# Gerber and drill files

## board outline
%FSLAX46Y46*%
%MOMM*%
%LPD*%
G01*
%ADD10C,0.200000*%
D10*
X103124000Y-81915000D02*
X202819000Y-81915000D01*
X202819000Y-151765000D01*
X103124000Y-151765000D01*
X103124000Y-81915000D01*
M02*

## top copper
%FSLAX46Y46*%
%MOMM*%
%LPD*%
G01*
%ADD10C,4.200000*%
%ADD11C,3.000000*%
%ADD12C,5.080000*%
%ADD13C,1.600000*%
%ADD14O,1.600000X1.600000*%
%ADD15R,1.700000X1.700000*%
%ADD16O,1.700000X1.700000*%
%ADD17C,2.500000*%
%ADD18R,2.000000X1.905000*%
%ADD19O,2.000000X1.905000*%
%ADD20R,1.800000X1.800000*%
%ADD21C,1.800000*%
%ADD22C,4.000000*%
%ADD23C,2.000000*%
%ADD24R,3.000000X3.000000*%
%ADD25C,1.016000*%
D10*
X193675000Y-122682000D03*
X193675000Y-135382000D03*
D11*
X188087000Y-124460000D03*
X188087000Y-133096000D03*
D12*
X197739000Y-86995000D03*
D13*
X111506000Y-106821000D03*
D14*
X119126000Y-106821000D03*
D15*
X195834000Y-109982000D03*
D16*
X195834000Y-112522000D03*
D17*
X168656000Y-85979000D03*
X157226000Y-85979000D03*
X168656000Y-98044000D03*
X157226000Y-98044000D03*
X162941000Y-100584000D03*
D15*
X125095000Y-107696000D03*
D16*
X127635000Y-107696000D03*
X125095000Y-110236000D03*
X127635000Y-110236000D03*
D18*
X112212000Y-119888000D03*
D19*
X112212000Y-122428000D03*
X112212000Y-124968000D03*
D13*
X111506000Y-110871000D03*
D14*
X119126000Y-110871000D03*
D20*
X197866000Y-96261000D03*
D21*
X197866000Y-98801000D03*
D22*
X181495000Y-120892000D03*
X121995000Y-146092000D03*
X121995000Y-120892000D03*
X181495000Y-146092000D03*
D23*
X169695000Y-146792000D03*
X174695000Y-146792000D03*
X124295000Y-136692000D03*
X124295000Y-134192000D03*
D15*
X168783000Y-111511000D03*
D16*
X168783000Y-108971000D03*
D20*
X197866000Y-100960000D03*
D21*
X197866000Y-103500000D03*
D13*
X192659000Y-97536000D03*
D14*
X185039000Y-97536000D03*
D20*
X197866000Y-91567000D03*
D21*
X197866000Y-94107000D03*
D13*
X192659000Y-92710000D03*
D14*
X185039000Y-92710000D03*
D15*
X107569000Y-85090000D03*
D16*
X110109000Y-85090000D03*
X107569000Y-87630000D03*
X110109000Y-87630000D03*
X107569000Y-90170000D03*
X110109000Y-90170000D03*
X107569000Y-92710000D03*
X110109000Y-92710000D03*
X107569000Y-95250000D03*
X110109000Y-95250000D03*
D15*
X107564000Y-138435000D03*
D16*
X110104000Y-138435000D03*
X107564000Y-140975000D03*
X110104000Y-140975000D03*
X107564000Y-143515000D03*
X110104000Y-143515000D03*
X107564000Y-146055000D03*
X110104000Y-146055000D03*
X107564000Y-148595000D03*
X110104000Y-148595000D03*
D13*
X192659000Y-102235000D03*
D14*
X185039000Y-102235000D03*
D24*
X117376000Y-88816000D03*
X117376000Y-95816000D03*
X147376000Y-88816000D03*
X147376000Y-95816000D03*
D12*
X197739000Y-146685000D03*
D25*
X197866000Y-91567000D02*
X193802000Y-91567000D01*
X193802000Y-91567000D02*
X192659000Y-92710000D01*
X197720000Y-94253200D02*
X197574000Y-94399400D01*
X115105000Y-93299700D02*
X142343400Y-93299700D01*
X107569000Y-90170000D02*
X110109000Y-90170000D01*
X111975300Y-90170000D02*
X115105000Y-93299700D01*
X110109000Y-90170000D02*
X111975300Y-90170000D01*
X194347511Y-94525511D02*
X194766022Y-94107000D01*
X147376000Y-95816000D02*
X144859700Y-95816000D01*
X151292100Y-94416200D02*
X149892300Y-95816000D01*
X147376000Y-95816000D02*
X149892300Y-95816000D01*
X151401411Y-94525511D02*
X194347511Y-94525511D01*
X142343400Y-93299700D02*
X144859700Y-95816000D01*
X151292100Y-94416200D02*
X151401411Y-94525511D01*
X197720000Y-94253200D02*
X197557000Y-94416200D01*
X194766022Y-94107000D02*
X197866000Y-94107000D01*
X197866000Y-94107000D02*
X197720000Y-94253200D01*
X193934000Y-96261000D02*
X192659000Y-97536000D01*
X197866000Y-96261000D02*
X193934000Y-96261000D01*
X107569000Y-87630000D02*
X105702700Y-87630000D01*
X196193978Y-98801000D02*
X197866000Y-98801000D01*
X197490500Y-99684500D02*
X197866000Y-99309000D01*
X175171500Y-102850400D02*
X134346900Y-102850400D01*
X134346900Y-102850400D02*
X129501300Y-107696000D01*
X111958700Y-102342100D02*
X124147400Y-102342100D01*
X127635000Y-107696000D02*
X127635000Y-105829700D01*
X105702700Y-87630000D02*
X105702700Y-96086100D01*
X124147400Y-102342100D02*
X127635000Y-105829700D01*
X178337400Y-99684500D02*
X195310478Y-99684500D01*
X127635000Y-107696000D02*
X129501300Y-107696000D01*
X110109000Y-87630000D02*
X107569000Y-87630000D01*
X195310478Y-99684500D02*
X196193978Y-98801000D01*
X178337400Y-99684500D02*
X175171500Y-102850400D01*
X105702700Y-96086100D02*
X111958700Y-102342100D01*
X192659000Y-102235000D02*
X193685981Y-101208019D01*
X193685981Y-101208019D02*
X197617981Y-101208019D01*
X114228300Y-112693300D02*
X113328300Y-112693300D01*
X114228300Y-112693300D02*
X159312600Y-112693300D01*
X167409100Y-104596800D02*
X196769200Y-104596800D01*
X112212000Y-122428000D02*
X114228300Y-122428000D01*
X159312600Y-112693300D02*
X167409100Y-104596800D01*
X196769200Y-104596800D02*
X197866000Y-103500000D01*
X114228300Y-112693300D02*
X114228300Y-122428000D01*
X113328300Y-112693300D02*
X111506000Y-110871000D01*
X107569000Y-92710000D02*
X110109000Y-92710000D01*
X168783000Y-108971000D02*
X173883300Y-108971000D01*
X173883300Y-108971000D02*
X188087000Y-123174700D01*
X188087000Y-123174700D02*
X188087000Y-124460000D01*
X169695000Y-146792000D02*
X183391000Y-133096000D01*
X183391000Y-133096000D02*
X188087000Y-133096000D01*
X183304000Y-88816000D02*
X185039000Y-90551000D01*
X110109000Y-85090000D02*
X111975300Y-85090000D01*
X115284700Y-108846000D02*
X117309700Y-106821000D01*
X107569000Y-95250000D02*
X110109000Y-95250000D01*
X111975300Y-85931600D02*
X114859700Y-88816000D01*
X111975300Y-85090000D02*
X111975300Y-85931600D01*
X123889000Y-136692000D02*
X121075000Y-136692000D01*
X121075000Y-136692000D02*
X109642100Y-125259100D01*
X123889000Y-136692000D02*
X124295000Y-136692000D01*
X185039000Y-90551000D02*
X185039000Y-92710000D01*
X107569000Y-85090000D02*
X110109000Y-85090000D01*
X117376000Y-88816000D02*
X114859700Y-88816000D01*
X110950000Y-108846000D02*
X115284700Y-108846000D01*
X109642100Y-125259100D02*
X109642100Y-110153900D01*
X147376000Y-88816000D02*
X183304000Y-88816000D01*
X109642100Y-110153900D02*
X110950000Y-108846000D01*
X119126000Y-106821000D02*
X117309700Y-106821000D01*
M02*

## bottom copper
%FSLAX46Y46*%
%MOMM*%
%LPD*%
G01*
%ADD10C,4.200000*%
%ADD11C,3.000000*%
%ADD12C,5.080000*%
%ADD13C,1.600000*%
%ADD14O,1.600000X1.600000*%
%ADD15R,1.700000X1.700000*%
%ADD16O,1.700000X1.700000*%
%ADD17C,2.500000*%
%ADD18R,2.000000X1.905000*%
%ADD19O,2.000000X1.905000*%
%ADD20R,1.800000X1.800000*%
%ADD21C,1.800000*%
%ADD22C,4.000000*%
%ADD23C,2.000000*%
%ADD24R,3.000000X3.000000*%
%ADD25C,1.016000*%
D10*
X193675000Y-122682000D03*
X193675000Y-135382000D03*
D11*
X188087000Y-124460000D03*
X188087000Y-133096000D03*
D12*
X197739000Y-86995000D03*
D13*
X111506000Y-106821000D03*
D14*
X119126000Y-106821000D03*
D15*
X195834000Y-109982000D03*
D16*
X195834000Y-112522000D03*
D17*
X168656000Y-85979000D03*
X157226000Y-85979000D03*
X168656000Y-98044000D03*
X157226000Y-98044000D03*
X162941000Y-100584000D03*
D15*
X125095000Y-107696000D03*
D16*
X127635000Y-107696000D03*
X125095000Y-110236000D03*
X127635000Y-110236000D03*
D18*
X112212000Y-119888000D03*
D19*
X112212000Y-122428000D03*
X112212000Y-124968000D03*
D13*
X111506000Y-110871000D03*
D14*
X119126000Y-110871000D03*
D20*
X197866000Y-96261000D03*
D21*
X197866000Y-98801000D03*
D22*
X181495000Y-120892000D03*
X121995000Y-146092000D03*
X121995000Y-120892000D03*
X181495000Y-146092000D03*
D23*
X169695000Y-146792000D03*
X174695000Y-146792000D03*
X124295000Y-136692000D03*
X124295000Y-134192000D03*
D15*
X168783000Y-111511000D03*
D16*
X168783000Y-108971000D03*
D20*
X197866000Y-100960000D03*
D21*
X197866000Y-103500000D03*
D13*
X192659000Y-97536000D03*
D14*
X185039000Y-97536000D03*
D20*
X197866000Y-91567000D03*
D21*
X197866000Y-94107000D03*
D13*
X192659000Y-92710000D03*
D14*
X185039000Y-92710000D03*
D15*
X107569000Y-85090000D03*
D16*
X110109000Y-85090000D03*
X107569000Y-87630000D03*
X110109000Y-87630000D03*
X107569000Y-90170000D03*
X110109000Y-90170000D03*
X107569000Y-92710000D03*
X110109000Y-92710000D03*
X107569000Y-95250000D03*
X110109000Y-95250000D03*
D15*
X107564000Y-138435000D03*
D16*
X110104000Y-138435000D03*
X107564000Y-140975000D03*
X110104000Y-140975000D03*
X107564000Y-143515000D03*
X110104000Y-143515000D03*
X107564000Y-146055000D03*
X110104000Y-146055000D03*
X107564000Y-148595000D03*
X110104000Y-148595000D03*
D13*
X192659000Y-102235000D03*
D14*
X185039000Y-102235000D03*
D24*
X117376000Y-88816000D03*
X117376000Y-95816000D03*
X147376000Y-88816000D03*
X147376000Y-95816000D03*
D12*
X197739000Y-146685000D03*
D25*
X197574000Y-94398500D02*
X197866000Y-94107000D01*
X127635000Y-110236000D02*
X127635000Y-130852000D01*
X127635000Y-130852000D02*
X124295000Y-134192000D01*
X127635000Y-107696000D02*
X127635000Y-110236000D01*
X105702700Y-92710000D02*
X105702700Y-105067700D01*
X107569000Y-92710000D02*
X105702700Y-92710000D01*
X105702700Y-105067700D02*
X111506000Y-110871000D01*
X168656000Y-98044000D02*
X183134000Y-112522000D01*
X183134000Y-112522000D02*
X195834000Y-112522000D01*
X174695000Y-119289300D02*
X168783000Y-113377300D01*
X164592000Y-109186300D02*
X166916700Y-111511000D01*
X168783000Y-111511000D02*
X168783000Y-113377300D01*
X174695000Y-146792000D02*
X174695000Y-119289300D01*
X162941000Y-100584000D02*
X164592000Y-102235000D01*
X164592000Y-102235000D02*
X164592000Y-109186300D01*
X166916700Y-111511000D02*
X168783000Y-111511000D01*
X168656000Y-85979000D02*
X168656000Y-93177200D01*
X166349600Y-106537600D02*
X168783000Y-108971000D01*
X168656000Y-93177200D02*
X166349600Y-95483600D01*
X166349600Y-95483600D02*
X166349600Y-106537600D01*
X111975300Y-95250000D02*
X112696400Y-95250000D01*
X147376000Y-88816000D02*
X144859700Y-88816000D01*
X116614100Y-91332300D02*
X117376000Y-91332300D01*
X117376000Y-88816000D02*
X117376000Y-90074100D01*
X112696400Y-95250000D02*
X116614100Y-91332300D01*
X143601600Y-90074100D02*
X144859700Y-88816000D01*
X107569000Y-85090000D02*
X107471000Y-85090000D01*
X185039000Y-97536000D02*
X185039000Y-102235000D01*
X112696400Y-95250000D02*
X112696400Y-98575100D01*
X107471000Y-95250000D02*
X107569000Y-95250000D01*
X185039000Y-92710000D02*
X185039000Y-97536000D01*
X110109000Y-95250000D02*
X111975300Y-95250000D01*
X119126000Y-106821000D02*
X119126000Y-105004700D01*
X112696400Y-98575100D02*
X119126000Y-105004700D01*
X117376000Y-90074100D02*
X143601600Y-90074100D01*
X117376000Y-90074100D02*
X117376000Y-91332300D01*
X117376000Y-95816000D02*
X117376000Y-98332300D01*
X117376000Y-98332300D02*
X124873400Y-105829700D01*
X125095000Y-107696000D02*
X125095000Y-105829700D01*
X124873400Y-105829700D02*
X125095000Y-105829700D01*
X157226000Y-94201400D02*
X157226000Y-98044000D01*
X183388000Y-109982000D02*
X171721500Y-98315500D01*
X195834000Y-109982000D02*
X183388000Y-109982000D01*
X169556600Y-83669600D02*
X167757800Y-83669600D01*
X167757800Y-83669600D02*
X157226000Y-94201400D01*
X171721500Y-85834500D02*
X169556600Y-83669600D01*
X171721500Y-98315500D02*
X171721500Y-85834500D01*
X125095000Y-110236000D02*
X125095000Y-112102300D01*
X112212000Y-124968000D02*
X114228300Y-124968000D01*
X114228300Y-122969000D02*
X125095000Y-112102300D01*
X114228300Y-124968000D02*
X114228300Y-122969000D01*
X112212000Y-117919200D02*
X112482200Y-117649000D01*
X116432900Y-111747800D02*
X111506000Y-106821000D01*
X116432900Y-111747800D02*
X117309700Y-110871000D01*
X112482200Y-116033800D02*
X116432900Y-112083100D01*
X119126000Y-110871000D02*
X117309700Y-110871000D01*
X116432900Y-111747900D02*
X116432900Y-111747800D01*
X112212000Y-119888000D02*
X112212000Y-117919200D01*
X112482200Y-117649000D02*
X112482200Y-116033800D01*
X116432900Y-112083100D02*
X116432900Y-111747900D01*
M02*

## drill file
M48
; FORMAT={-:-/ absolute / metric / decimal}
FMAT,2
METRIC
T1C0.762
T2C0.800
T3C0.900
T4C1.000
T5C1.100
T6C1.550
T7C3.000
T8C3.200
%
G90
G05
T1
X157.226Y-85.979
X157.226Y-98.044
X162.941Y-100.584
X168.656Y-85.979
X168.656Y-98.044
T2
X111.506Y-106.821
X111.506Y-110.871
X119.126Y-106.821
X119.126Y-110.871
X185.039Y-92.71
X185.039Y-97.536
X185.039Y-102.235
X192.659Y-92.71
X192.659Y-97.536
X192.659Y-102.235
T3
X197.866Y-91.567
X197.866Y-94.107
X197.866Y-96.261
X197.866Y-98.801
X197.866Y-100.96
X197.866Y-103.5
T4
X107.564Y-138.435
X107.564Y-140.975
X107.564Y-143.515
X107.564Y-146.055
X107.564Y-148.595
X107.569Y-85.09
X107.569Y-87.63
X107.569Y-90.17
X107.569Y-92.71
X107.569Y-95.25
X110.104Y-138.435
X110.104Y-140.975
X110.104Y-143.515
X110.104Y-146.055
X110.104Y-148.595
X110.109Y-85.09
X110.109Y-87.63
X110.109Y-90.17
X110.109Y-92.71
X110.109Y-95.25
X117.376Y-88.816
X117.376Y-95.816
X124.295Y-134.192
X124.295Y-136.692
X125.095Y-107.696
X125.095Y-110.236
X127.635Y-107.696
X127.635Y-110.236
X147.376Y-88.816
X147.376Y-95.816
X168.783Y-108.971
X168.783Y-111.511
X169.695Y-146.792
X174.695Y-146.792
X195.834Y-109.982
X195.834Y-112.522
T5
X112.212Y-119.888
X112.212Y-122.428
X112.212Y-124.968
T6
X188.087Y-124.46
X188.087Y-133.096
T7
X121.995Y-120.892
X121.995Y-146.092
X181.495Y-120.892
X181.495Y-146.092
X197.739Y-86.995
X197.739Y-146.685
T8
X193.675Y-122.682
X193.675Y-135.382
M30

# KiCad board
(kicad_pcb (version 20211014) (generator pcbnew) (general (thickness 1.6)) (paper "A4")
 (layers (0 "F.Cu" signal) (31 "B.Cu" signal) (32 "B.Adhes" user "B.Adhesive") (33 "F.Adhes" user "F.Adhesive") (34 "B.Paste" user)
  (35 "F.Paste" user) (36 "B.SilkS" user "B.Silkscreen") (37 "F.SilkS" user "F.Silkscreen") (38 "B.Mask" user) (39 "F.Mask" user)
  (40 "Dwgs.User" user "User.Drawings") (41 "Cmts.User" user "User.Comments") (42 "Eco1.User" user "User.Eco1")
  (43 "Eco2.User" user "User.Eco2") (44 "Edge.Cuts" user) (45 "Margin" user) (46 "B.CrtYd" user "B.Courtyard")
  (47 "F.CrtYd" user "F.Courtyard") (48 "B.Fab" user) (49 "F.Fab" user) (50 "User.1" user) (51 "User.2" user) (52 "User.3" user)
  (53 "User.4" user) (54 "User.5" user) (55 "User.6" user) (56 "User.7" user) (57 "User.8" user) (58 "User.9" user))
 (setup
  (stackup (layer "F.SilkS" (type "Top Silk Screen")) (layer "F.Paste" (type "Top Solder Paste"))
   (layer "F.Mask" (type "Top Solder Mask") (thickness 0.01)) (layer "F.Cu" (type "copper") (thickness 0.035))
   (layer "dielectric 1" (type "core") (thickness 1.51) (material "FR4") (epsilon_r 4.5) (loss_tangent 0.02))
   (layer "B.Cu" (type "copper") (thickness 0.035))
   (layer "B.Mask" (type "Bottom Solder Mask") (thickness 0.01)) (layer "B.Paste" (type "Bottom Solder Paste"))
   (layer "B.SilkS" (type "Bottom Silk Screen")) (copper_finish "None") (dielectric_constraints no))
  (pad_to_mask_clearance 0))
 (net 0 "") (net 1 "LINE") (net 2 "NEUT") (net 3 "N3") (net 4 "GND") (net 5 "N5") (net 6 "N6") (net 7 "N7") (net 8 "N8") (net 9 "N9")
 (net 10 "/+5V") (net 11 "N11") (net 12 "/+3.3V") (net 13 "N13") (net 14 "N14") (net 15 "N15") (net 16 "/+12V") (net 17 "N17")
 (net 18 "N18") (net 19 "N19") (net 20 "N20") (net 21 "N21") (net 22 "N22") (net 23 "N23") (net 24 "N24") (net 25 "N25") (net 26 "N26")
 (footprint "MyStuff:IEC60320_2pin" (layer "F.Cu") (at 188.595 117.856 -90)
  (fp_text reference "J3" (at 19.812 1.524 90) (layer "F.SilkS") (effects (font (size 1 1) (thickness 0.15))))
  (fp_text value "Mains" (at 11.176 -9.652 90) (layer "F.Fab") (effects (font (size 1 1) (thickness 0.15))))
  (pad "" thru_hole circle locked (at 4.826 -5.08 270) (size 4.2 4.2) (drill 3.2) (layers *.Cu *.Mask))
  (pad "" thru_hole circle locked (at 17.526 -5.08 270) (size 4.2 4.2) (drill 3.2) (layers *.Cu *.Mask))
  (pad "1" thru_hole circle locked (at 6.604 0.508 270) (size 3 3) (drill 1.55) (layers *.Cu *.Mask) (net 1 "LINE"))
  (pad "2" thru_hole circle locked (at 15.24 0.508 270) (size 3 3) (drill 1.55) (layers *.Cu *.Mask) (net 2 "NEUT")))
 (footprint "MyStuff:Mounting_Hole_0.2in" (layer "F.Cu") (at 197.739 86.995)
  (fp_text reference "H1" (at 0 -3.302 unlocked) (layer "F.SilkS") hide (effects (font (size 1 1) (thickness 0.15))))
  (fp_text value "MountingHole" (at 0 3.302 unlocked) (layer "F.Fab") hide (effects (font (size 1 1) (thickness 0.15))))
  (pad "" thru_hole circle (at 0 0) (size 5.08 5.08) (drill 3) (layers *.Cu *.Mask)))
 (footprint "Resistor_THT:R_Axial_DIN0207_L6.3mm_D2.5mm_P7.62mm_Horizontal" (layer "F.Cu") (at 111.506 106.821)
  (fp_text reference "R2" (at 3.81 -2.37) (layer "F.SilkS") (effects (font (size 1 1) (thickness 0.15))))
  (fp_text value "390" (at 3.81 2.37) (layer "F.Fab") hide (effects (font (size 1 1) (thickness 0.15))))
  (pad "1" thru_hole circle (at 0 0) (size 1.6 1.6) (drill 0.8) (layers *.Cu *.Mask) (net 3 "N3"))
  (pad "2" thru_hole oval (at 7.62 0) (size 1.6 1.6) (drill 0.8) (layers *.Cu *.Mask) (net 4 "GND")))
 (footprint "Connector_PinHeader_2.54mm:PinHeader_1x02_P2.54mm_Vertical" (layer "F.Cu") (at 195.834 109.982)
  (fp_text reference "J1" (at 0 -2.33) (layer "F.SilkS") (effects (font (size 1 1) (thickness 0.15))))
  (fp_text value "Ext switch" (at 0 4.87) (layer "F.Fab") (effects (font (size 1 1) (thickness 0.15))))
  (pad "1" thru_hole rect (at 0 0) (size 1.7 1.7) (drill 1) (layers *.Cu *.Mask) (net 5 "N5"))
  (pad "2" thru_hole oval (at 0 2.54) (size 1.7 1.7) (drill 1) (layers *.Cu *.Mask) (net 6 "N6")))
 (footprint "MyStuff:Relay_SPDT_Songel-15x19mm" (layer "F.Cu") (at 168.656 85.979 180)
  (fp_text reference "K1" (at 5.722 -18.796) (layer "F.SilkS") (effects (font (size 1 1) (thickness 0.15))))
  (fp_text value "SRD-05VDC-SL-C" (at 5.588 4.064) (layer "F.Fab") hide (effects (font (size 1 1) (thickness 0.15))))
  (pad "1" thru_hole circle locked (at 0 0 180) (size 2.5 2.5) (drill 0.762) (layers *.Cu *.Mask) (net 1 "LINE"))
  (pad "2" thru_hole circle locked (at 11.43 0 180) (size 2.5 2.5) (drill 0.762) (layers *.Cu *.Mask) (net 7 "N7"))
  (pad "3" thru_hole circle locked (at 0 -12.065 180) (size 2.5 2.5) (drill 0.762) (layers *.Cu *.Mask) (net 6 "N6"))
  (pad "4" thru_hole circle locked (at 11.43 -12.065 180) (size 2.5 2.5) (drill 0.762) (layers *.Cu *.Mask) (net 5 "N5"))
  (pad "5" thru_hole circle locked (at 5.715 -14.605 180) (size 2.5 2.5) (drill 0.762) (layers *.Cu *.Mask) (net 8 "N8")))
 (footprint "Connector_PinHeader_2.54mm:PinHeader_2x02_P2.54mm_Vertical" (layer "F.Cu") (at 125.095 107.696)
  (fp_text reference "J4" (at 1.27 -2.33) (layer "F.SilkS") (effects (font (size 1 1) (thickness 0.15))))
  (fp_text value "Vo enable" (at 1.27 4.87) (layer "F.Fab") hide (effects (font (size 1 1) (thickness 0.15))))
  (pad "1" thru_hole rect (at 0 0) (size 1.7 1.7) (drill 1) (layers *.Cu *.Mask) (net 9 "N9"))
  (pad "2" thru_hole oval (at 2.54 0) (size 1.7 1.7) (drill 1) (layers *.Cu *.Mask) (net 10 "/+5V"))
  (pad "3" thru_hole oval (at 0 2.54) (size 1.7 1.7) (drill 1) (layers *.Cu *.Mask) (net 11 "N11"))
  (pad "4" thru_hole oval (at 2.54 2.54) (size 1.7 1.7) (drill 1) (layers *.Cu *.Mask) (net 10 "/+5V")))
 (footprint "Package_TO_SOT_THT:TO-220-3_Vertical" (layer "F.Cu") (at 112.212 119.888 -90)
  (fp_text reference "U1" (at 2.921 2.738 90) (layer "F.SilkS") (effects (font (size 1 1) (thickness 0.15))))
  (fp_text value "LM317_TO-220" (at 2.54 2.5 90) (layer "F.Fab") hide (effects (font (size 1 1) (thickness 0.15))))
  (pad "1" thru_hole rect (at 0 0 270) (size 1.905 2) (drill 1.1) (layers *.Cu *.Mask) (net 3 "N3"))
  (pad "2" thru_hole oval (at 2.54 0 270) (size 1.905 2) (drill 1.1) (layers *.Cu *.Mask) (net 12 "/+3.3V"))
  (pad "3" thru_hole oval (at 5.08 0 270) (size 1.905 2) (drill 1.1) (layers *.Cu *.Mask) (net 11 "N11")))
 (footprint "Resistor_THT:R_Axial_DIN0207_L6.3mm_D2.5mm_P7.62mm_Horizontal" (layer "F.Cu") (at 111.506 110.871)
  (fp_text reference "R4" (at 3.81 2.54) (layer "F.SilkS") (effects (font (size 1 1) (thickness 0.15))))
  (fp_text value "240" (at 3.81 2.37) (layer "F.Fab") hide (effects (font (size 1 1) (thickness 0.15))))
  (pad "1" thru_hole circle (at 0 0) (size 1.6 1.6) (drill 0.8) (layers *.Cu *.Mask) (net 12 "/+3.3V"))
  (pad "2" thru_hole oval (at 7.62 0) (size 1.6 1.6) (drill 0.8) (layers *.Cu *.Mask) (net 3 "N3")))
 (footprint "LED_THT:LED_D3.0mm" (layer "F.Cu") (at 197.866 96.261 -90)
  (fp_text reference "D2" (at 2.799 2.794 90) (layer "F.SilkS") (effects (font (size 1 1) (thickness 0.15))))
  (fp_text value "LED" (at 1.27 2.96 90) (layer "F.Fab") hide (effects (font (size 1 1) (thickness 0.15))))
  (pad "1" thru_hole rect (at 0 0 270) (size 1.8 1.8) (drill 0.9) (layers *.Cu *.Mask) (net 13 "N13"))
  (pad "2" thru_hole circle (at 2.54 0 270) (size 1.8 1.8) (drill 0.9) (layers *.Cu *.Mask) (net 10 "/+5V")))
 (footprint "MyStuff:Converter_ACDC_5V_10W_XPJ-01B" (layer "F.Cu") (at 183.995 149.892 90)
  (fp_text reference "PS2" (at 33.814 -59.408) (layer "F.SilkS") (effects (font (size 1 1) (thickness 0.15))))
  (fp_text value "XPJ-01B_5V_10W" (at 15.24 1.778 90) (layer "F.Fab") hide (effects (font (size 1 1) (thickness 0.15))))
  (pad "" thru_hole circle locked (at 29 -2.5 90) (size 4 4) (drill 3) (layers *.Cu *.Mask))
  (pad "" thru_hole circle locked (at 3.8 -62 90) (size 4 4) (drill 3) (layers *.Cu *.Mask))
  (pad "" thru_hole circle locked (at 29 -62 90) (size 4 4) (drill 3) (layers *.Cu *.Mask))
  (pad "" thru_hole circle locked (at 3.8 -2.5 90) (size 4 4) (drill 3) (layers *.Cu *.Mask))
  (pad "1" thru_hole circle locked (at 3.1 -14.3 90) (size 2 2) (drill 1) (layers *.Cu *.Mask) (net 2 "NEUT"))
  (pad "2" thru_hole circle locked (at 3.1 -9.3 90) (size 2 2) (drill 1) (layers *.Cu *.Mask) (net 8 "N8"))
  (pad "3" thru_hole circle locked (at 13.2 -59.7 90) (size 2 2) (drill 1) (layers *.Cu *.Mask) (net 4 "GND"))
  (pad "4" thru_hole circle locked (at 15.7 -59.7 90) (size 2 2) (drill 1) (layers *.Cu *.Mask) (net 10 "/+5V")))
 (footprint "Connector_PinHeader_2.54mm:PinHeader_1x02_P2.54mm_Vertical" (layer "F.Cu") (at 168.783 111.511 180)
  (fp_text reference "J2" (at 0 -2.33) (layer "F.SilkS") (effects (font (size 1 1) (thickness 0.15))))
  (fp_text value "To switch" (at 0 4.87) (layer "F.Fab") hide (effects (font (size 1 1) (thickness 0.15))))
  (pad "1" thru_hole rect (at 0 0 180) (size 1.7 1.7) (drill 1) (layers *.Cu *.Mask) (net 8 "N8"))
  (pad "2" thru_hole oval (at 0 2.54 180) (size 1.7 1.7) (drill 1) (layers *.Cu *.Mask) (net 1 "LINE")))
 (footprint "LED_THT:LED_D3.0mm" (layer "F.Cu") (at 197.866 100.96 -90)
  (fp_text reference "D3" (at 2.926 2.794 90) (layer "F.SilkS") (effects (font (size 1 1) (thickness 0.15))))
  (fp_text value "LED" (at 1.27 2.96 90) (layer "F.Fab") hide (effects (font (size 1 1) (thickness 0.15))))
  (pad "1" thru_hole rect (at 0 0 270) (size 1.8 1.8) (drill 0.9) (layers *.Cu *.Mask) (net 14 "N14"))
  (pad "2" thru_hole circle (at 2.54 0 270) (size 1.8 1.8) (drill 0.9) (layers *.Cu *.Mask) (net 12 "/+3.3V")))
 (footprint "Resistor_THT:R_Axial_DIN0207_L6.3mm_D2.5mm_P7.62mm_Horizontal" (layer "F.Cu") (at 192.659 97.536 180)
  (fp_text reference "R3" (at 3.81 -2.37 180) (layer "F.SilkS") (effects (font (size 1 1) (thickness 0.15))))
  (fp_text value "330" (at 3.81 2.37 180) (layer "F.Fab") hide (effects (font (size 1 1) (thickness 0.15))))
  (pad "1" thru_hole circle (at 0 0 180) (size 1.6 1.6) (drill 0.8) (layers *.Cu *.Mask) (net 13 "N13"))
  (pad "2" thru_hole oval (at 7.62 0 180) (size 1.6 1.6) (drill 0.8) (layers *.Cu *.Mask) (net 4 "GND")))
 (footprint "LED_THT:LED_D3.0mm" (layer "F.Cu") (at 197.866 91.567 -90)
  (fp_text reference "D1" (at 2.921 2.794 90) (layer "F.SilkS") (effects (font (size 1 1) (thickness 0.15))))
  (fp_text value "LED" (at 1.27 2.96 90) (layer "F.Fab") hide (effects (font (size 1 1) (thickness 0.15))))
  (pad "1" thru_hole rect (at 0 0 270) (size 1.8 1.8) (drill 0.9) (layers *.Cu *.Mask) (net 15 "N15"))
  (pad "2" thru_hole circle (at 2.54 0 270) (size 1.8 1.8) (drill 0.9) (layers *.Cu *.Mask) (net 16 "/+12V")))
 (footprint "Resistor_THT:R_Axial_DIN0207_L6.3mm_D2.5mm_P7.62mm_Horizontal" (layer "F.Cu") (at 192.659 92.71 180)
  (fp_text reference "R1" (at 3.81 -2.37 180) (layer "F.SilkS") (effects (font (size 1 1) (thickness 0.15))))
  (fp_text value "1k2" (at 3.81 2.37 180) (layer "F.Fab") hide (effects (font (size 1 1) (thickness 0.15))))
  (pad "1" thru_hole circle (at 0 0 180) (size 1.6 1.6) (drill 0.8) (layers *.Cu *.Mask) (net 15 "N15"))
  (pad "2" thru_hole oval (at 7.62 0 180) (size 1.6 1.6) (drill 0.8) (layers *.Cu *.Mask) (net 4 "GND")))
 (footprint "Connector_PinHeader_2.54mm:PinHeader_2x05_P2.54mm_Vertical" (layer "F.Cu") (at 107.569 85.09)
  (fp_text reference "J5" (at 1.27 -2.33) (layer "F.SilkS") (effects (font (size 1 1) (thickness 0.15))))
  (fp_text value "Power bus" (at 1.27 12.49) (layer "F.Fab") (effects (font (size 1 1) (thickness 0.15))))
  (pad "1" thru_hole rect (at 0 0) (size 1.7 1.7) (drill 1) (layers *.Cu *.Mask) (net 4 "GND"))
  (pad "2" thru_hole oval (at 2.54 0) (size 1.7 1.7) (drill 1) (layers *.Cu *.Mask) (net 4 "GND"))
  (pad "3" thru_hole oval (at 0 2.54) (size 1.7 1.7) (drill 1) (layers *.Cu *.Mask) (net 10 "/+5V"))
  (pad "4" thru_hole oval (at 2.54 2.54) (size 1.7 1.7) (drill 1) (layers *.Cu *.Mask) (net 10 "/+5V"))
  (pad "5" thru_hole oval (at 0 5.08) (size 1.7 1.7) (drill 1) (layers *.Cu *.Mask) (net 16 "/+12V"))
  (pad "6" thru_hole oval (at 2.54 5.08) (size 1.7 1.7) (drill 1) (layers *.Cu *.Mask) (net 16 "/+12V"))
  (pad "7" thru_hole oval (at 0 7.62) (size 1.7 1.7) (drill 1) (layers *.Cu *.Mask) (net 12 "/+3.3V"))
  (pad "8" thru_hole oval (at 2.54 7.62) (size 1.7 1.7) (drill 1) (layers *.Cu *.Mask) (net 12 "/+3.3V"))
  (pad "9" thru_hole oval (at 0 10.16) (size 1.7 1.7) (drill 1) (layers *.Cu *.Mask) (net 4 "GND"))
  (pad "10" thru_hole oval (at 2.54 10.16) (size 1.7 1.7) (drill 1) (layers *.Cu *.Mask) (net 4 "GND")))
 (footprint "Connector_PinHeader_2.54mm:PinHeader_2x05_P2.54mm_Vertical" (layer "F.Cu") (at 107.564 138.435)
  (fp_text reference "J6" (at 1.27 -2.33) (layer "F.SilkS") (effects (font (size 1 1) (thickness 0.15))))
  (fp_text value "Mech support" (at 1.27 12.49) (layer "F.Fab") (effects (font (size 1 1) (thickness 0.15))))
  (pad "1" thru_hole rect (at 0 0) (size 1.7 1.7) (drill 1) (layers *.Cu *.Mask) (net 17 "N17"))
  (pad "2" thru_hole oval (at 2.54 0) (size 1.7 1.7) (drill 1) (layers *.Cu *.Mask) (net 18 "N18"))
  (pad "3" thru_hole oval (at 0 2.54) (size 1.7 1.7) (drill 1) (layers *.Cu *.Mask) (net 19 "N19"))
  (pad "4" thru_hole oval (at 2.54 2.54) (size 1.7 1.7) (drill 1) (layers *.Cu *.Mask) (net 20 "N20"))
  (pad "5" thru_hole oval (at 0 5.08) (size 1.7 1.7) (drill 1) (layers *.Cu *.Mask) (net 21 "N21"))
  (pad "6" thru_hole oval (at 2.54 5.08) (size 1.7 1.7) (drill 1) (layers *.Cu *.Mask) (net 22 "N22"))
  (pad "7" thru_hole oval (at 0 7.62) (size 1.7 1.7) (drill 1) (layers *.Cu *.Mask) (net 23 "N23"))
  (pad "8" thru_hole oval (at 2.54 7.62) (size 1.7 1.7) (drill 1) (layers *.Cu *.Mask) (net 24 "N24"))
  (pad "9" thru_hole oval (at 0 10.16) (size 1.7 1.7) (drill 1) (layers *.Cu *.Mask) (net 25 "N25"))
  (pad "10" thru_hole oval (at 2.54 10.16) (size 1.7 1.7) (drill 1) (layers *.Cu *.Mask) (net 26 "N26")))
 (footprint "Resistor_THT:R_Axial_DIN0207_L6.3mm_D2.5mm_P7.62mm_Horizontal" (layer "F.Cu") (at 192.659 102.235 180)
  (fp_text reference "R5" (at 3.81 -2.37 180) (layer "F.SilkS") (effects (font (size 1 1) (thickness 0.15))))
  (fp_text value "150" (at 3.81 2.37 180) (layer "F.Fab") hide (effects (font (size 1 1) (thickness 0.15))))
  (pad "1" thru_hole circle (at 0 0 180) (size 1.6 1.6) (drill 0.8) (layers *.Cu *.Mask) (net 14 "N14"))
  (pad "2" thru_hole oval (at 7.62 0 180) (size 1.6 1.6) (drill 0.8) (layers *.Cu *.Mask) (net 4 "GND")))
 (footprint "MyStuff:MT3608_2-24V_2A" (layer "F.Cu") (at 150.876 83.566 180)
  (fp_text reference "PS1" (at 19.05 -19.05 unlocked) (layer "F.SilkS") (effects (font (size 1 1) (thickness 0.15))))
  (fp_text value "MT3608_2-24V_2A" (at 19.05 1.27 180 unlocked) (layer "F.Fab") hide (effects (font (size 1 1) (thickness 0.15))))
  (pad "1" thru_hole rect (at 33.5 -5.25 180) (size 3 3) (drill 1) (layers *.Cu *.Mask) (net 4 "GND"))
  (pad "2" thru_hole rect (at 33.5 -12.25 180) (size 3 3) (drill 1) (layers *.Cu *.Mask) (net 9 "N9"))
  (pad "3" thru_hole rect (at 3.5 -5.25 180) (size 3 3) (drill 1) (layers *.Cu *.Mask) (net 4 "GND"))
  (pad "4" thru_hole rect (at 3.5 -12.25 180) (size 3 3) (drill 1) (layers *.Cu *.Mask) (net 16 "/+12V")))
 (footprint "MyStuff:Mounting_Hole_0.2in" (layer "F.Cu") (at 197.739 146.685)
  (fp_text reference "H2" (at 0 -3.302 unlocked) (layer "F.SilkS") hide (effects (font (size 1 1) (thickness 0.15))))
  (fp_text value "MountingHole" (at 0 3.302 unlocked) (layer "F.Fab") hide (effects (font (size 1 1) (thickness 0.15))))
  (pad "" thru_hole circle (at 0 0) (size 5.08 5.08) (drill 3) (layers *.Cu *.Mask)))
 (gr_rect (start 103.124 81.915) (end 202.819 151.765) (layer "Edge.Cuts") (width 0.2) (fill none))
 (segment (start 197.866 91.567) (end 193.802 91.567) (width 1.016) (layer "F.Cu") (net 15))
 (segment (start 193.802 91.567) (end 192.659 92.71) (width 1.016) (layer "F.Cu") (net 15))
 (segment (start 197.72 94.2532) (end 197.574 94.3994) (width 1.016) (layer "F.Cu") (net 16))
 (segment (start 115.105 93.2997) (end 142.3434 93.2997) (width 1.016) (layer "F.Cu") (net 16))
 (segment (start 107.569 90.17) (end 110.109 90.17) (width 1.016) (layer "F.Cu") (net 16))
 (segment (start 111.9753 90.17) (end 115.105 93.2997) (width 1.016) (layer "F.Cu") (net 16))
 (segment (start 110.109 90.17) (end 111.9753 90.17) (width 1.016) (layer "F.Cu") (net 16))
 (segment (start 194.347511 94.525511) (end 194.766022 94.107) (width 1.016) (layer "F.Cu") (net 16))
 (segment (start 147.376 95.816) (end 144.8597 95.816) (width 1.016) (layer "F.Cu") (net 16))
 (segment (start 151.2921 94.4162) (end 149.8923 95.816) (width 1.016) (layer "F.Cu") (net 16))
 (segment (start 147.376 95.816) (end 149.8923 95.816) (width 1.016) (layer "F.Cu") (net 16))
 (segment (start 151.401411 94.525511) (end 194.347511 94.525511) (width 1.016) (layer "F.Cu") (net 16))
 (segment (start 142.3434 93.2997) (end 144.8597 95.816) (width 1.016) (layer "F.Cu") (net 16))
 (segment (start 151.2921 94.4162) (end 151.401411 94.525511) (width 1.016) (layer "F.Cu") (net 16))
 (segment (start 197.72 94.2532) (end 197.557 94.4162) (width 1.016) (layer "F.Cu") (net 16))
 (segment (start 194.766022 94.107) (end 197.866 94.107) (width 1.016) (layer "F.Cu") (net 16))
 (segment (start 197.866 94.107) (end 197.72 94.2532) (width 1.016) (layer "F.Cu") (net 16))
 (segment (start 197.574 94.3985) (end 197.866 94.107) (width 1.016) (layer "B.Cu") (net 16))
 (segment (start 193.934 96.261) (end 192.659 97.536) (width 1.016) (layer "F.Cu") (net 13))
 (segment (start 197.866 96.261) (end 193.934 96.261) (width 1.016) (layer "F.Cu") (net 13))
 (segment (start 107.569 87.63) (end 105.7027 87.63) (width 1.016) (layer "F.Cu") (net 10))
 (segment (start 196.193978 98.801) (end 197.866 98.801) (width 1.016) (layer "F.Cu") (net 10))
 (segment (start 197.4905 99.6845) (end 197.866 99.309) (width 1.016) (layer "F.Cu") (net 10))
 (segment (start 175.1715 102.8504) (end 134.3469 102.8504) (width 1.016) (layer "F.Cu") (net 10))
 (segment (start 134.3469 102.8504) (end 129.5013 107.696) (width 1.016) (layer "F.Cu") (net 10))
 (segment (start 111.9587 102.3421) (end 124.1474 102.3421) (width 1.016) (layer "F.Cu") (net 10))
 (segment (start 127.635 107.696) (end 127.635 105.8297) (width 1.016) (layer "F.Cu") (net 10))
 (segment (start 105.7027 87.63) (end 105.7027 96.0861) (width 1.016) (layer "F.Cu") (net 10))
 (segment (start 124.1474 102.3421) (end 127.635 105.8297) (width 1.016) (layer "F.Cu") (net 10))
 (segment (start 178.3374 99.6845) (end 195.310478 99.6845) (width 1.016) (layer "F.Cu") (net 10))
 (segment (start 127.635 107.696) (end 129.5013 107.696) (width 1.016) (layer "F.Cu") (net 10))
 (segment (start 110.109 87.63) (end 107.569 87.63) (width 1.016) (layer "F.Cu") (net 10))
 (segment (start 195.310478 99.6845) (end 196.193978 98.801) (width 1.016) (layer "F.Cu") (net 10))
 (segment (start 178.3374 99.6845) (end 175.1715 102.8504) (width 1.016) (layer "F.Cu") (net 10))
 (segment (start 105.7027 96.0861) (end 111.9587 102.3421) (width 1.016) (layer "F.Cu") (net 10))
 (segment (start 127.635 110.236) (end 127.635 130.852) (width 1.016) (layer "B.Cu") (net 10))
 (segment (start 127.635 130.852) (end 124.295 134.192) (width 1.016) (layer "B.Cu") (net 10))
 (segment (start 127.635 107.696) (end 127.635 110.236) (width 1.016) (layer "B.Cu") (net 10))
 (segment (start 192.659 102.235) (end 193.685981 101.208019) (width 1.016) (layer "F.Cu") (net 14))
 (segment (start 193.685981 101.208019) (end 197.617981 101.208019) (width 1.016) (layer "F.Cu") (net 14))
 (segment (start 114.2283 112.6933) (end 113.3283 112.6933) (width 1.016) (layer "F.Cu") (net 12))
 (segment (start 114.2283 112.6933) (end 159.3126 112.6933) (width 1.016) (layer "F.Cu") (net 12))
 (segment (start 167.4091 104.5968) (end 196.7692 104.5968) (width 1.016) (layer "F.Cu") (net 12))
 (segment (start 112.212 122.428) (end 114.2283 122.428) (width 1.016) (layer "F.Cu") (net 12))
 (segment (start 159.3126 112.6933) (end 167.4091 104.5968) (width 1.016) (layer "F.Cu") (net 12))
 (segment (start 196.7692 104.5968) (end 197.866 103.5) (width 1.016) (layer "F.Cu") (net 12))
 (segment (start 114.2283 112.6933) (end 114.2283 122.428) (width 1.016) (layer "F.Cu") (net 12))
 (segment (start 113.3283 112.6933) (end 111.506 110.871) (width 1.016) (layer "F.Cu") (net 12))
 (segment (start 107.569 92.71) (end 110.109 92.71) (width 1.016) (layer "F.Cu") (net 12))
 (segment (start 105.7027 92.71) (end 105.7027 105.0677) (width 1.016) (layer "B.Cu") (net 12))
 (segment (start 107.569 92.71) (end 105.7027 92.71) (width 1.016) (layer "B.Cu") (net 12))
 (segment (start 105.7027 105.0677) (end 111.506 110.871) (width 1.016) (layer "B.Cu") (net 12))
 (segment (start 168.656 98.044) (end 183.134 112.522) (width 1.016) (layer "B.Cu") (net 6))
 (segment (start 183.134 112.522) (end 195.834 112.522) (width 1.016) (layer "B.Cu") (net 6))
 (segment (start 174.695 119.2893) (end 168.783 113.3773) (width 1.016) (layer "B.Cu") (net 8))
 (segment (start 164.592 109.1863) (end 166.9167 111.511) (width 1.016) (layer "B.Cu") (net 8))
 (segment (start 168.783 111.511) (end 168.783 113.3773) (width 1.016) (layer "B.Cu") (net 8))
 (segment (start 174.695 146.792) (end 174.695 119.2893) (width 1.016) (layer "B.Cu") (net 8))
 (segment (start 162.941 100.584) (end 164.592 102.235) (width 1.016) (layer "B.Cu") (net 8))
 (segment (start 164.592 102.235) (end 164.592 109.1863) (width 1.016) (layer "B.Cu") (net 8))
 (segment (start 166.9167 111.511) (end 168.783 111.511) (width 1.016) (layer "B.Cu") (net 8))
 (segment (start 168.783 108.971) (end 173.8833 108.971) (width 1.016) (layer "F.Cu") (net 1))
 (segment (start 173.8833 108.971) (end 188.087 123.1747) (width 1.016) (layer "F.Cu") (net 1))
 (segment (start 188.087 123.1747) (end 188.087 124.46) (width 1.016) (layer "F.Cu") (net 1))
 (segment (start 168.656 85.979) (end 168.656 93.1772) (width 1.016) (layer "B.Cu") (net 1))
 (segment (start 166.3496 106.5376) (end 168.783 108.971) (width 1.016) (layer "B.Cu") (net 1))
 (segment (start 168.656 93.1772) (end 166.3496 95.4836) (width 1.016) (layer "B.Cu") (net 1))
 (segment (start 166.3496 95.4836) (end 166.3496 106.5376) (width 1.016) (layer "B.Cu") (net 1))
 (segment (start 169.695 146.792) (end 183.391 133.096) (width 1.016) (layer "F.Cu") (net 2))
 (segment (start 183.391 133.096) (end 188.087 133.096) (width 1.016) (layer "F.Cu") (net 2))
 (segment (start 183.304 88.816) (end 185.039 90.551) (width 1.016) (layer "F.Cu") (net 4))
 (segment (start 110.109 85.09) (end 111.9753 85.09) (width 1.016) (layer "F.Cu") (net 4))
 (segment (start 115.2847 108.846) (end 117.3097 106.821) (width 1.016) (layer "F.Cu") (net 4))
 (segment (start 107.569 95.25) (end 110.109 95.25) (width 1.016) (layer "F.Cu") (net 4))
 (segment (start 111.9753 85.9316) (end 114.8597 88.816) (width 1.016) (layer "F.Cu") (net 4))
 (segment (start 111.9753 85.09) (end 111.9753 85.9316) (width 1.016) (layer "F.Cu") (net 4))
 (segment (start 123.889 136.692) (end 121.075 136.692) (width 1.016) (layer "F.Cu") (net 4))
 (segment (start 121.075 136.692) (end 109.6421 125.2591) (width 1.016) (layer "F.Cu") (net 4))
 (segment (start 123.889 136.692) (end 124.295 136.692) (width 1.016) (layer "F.Cu") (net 4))
 (segment (start 185.039 90.551) (end 185.039 92.71) (width 1.016) (layer "F.Cu") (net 4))
 (segment (start 107.569 85.09) (end 110.109 85.09) (width 1.016) (layer "F.Cu") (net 4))
 (segment (start 117.376 88.816) (end 114.8597 88.816) (width 1.016) (layer "F.Cu") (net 4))
 (segment (start 110.95 108.846) (end 115.2847 108.846) (width 1.016) (layer "F.Cu") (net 4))
 (segment (start 109.6421 125.2591) (end 109.6421 110.1539) (width 1.016) (layer "F.Cu") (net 4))
 (segment (start 147.376 88.816) (end 183.304 88.816) (width 1.016) (layer "F.Cu") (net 4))
 (segment (start 109.6421 110.1539) (end 110.95 108.846) (width 1.016) (layer "F.Cu") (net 4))
 (segment (start 119.126 106.821) (end 117.3097 106.821) (width 1.016) (layer "F.Cu") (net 4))
 (segment (start 111.9753 95.25) (end 112.6964 95.25) (width 1.016) (layer "B.Cu") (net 4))
 (segment (start 147.376 88.816) (end 144.8597 88.816) (width 1.016) (layer "B.Cu") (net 4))
 (segment (start 116.6141 91.3323) (end 117.376 91.3323) (width 1.016) (layer "B.Cu") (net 4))
 (segment (start 117.376 88.816) (end 117.376 90.0741) (width 1.016) (layer "B.Cu") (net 4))
 (segment (start 112.6964 95.25) (end 116.6141 91.3323) (width 1.016) (layer "B.Cu") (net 4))
 (segment (start 143.6016 90.0741) (end 144.8597 88.816) (width 1.016) (layer "B.Cu") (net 4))
 (segment (start 107.569 85.09) (end 107.471 85.09) (width 1.016) (layer "B.Cu") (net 4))
 (segment (start 185.039 97.536) (end 185.039 102.235) (width 1.016) (layer "B.Cu") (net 4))
 (segment (start 112.6964 95.25) (end 112.6964 98.5751) (width 1.016) (layer "B.Cu") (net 4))
 (segment (start 107.471 95.25) (end 107.569 95.25) (width 1.016) (layer "B.Cu") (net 4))
 (segment (start 185.039 92.71) (end 185.039 97.536) (width 1.016) (layer "B.Cu") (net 4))
 (segment (start 110.109 95.25) (end 111.9753 95.25) (width 1.016) (layer "B.Cu") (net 4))
 (segment (start 119.126 106.821) (end 119.126 105.0047) (width 1.016) (layer "B.Cu") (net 4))
 (segment (start 112.6964 98.5751) (end 119.126 105.0047) (width 1.016) (layer "B.Cu") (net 4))
 (segment (start 117.376 90.0741) (end 143.6016 90.0741) (width 1.016) (layer "B.Cu") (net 4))
 (segment (start 117.376 90.0741) (end 117.376 91.3323) (width 1.016) (layer "B.Cu") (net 4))
 (segment (start 117.376 95.816) (end 117.376 98.3323) (width 1.016) (layer "B.Cu") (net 9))
 (segment (start 117.376 98.3323) (end 124.8734 105.8297) (width 1.016) (layer "B.Cu") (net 9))
 (segment (start 125.095 107.696) (end 125.095 105.8297) (width 1.016) (layer "B.Cu") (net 9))
 (segment (start 124.8734 105.8297) (end 125.095 105.8297) (width 1.016) (layer "B.Cu") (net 9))
 (segment (start 157.226 94.2014) (end 157.226 98.044) (width 1.016) (layer "B.Cu") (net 5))
 (segment (start 183.388 109.982) (end 171.7215 98.3155) (width 1.016) (layer "B.Cu") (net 5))
 (segment (start 195.834 109.982) (end 183.388 109.982) (width 1.016) (layer "B.Cu") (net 5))
 (segment (start 169.5566 83.6696) (end 167.7578 83.6696) (width 1.016) (layer "B.Cu") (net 5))
 (segment (start 167.7578 83.6696) (end 157.226 94.2014) (width 1.016) (layer "B.Cu") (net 5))
 (segment (start 171.7215 85.8345) (end 169.5566 83.6696) (width 1.016) (layer "B.Cu") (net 5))
 (segment (start 171.7215 98.3155) (end 171.7215 85.8345) (width 1.016) (layer "B.Cu") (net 5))
 (segment (start 125.095 110.236) (end 125.095 112.1023) (width 1.016) (layer "B.Cu") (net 11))
 (segment (start 112.212 124.968) (end 114.2283 124.968) (width 1.016) (layer "B.Cu") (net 11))
 (segment (start 114.2283 122.969) (end 125.095 112.1023) (width 1.016) (layer "B.Cu") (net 11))
 (segment (start 114.2283 124.968) (end 114.2283 122.969) (width 1.016) (layer "B.Cu") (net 11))
 (segment (start 112.212 117.9192) (end 112.4822 117.649) (width 1.016) (layer "B.Cu") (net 3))
 (segment (start 116.4329 111.7478) (end 111.506 106.821) (width 1.016) (layer "B.Cu") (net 3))
 (segment (start 116.4329 111.7478) (end 117.3097 110.871) (width 1.016) (layer "B.Cu") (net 3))
 (segment (start 112.4822 116.0338) (end 116.4329 112.0831) (width 1.016) (layer "B.Cu") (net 3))
 (segment (start 119.126 110.871) (end 117.3097 110.871) (width 1.016) (layer "B.Cu") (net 3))
 (segment (start 116.4329 111.7479) (end 116.4329 111.7478) (width 1.016) (layer "B.Cu") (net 3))
 (segment (start 112.212 119.888) (end 112.212 117.9192) (width 1.016) (layer "B.Cu") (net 3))
 (segment (start 112.4822 117.649) (end 112.4822 116.0338) (width 1.016) (layer "B.Cu") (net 3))
 (segment (start 116.4329 112.0831) (end 116.4329 111.7479) (width 1.016) (layer "B.Cu") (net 3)))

